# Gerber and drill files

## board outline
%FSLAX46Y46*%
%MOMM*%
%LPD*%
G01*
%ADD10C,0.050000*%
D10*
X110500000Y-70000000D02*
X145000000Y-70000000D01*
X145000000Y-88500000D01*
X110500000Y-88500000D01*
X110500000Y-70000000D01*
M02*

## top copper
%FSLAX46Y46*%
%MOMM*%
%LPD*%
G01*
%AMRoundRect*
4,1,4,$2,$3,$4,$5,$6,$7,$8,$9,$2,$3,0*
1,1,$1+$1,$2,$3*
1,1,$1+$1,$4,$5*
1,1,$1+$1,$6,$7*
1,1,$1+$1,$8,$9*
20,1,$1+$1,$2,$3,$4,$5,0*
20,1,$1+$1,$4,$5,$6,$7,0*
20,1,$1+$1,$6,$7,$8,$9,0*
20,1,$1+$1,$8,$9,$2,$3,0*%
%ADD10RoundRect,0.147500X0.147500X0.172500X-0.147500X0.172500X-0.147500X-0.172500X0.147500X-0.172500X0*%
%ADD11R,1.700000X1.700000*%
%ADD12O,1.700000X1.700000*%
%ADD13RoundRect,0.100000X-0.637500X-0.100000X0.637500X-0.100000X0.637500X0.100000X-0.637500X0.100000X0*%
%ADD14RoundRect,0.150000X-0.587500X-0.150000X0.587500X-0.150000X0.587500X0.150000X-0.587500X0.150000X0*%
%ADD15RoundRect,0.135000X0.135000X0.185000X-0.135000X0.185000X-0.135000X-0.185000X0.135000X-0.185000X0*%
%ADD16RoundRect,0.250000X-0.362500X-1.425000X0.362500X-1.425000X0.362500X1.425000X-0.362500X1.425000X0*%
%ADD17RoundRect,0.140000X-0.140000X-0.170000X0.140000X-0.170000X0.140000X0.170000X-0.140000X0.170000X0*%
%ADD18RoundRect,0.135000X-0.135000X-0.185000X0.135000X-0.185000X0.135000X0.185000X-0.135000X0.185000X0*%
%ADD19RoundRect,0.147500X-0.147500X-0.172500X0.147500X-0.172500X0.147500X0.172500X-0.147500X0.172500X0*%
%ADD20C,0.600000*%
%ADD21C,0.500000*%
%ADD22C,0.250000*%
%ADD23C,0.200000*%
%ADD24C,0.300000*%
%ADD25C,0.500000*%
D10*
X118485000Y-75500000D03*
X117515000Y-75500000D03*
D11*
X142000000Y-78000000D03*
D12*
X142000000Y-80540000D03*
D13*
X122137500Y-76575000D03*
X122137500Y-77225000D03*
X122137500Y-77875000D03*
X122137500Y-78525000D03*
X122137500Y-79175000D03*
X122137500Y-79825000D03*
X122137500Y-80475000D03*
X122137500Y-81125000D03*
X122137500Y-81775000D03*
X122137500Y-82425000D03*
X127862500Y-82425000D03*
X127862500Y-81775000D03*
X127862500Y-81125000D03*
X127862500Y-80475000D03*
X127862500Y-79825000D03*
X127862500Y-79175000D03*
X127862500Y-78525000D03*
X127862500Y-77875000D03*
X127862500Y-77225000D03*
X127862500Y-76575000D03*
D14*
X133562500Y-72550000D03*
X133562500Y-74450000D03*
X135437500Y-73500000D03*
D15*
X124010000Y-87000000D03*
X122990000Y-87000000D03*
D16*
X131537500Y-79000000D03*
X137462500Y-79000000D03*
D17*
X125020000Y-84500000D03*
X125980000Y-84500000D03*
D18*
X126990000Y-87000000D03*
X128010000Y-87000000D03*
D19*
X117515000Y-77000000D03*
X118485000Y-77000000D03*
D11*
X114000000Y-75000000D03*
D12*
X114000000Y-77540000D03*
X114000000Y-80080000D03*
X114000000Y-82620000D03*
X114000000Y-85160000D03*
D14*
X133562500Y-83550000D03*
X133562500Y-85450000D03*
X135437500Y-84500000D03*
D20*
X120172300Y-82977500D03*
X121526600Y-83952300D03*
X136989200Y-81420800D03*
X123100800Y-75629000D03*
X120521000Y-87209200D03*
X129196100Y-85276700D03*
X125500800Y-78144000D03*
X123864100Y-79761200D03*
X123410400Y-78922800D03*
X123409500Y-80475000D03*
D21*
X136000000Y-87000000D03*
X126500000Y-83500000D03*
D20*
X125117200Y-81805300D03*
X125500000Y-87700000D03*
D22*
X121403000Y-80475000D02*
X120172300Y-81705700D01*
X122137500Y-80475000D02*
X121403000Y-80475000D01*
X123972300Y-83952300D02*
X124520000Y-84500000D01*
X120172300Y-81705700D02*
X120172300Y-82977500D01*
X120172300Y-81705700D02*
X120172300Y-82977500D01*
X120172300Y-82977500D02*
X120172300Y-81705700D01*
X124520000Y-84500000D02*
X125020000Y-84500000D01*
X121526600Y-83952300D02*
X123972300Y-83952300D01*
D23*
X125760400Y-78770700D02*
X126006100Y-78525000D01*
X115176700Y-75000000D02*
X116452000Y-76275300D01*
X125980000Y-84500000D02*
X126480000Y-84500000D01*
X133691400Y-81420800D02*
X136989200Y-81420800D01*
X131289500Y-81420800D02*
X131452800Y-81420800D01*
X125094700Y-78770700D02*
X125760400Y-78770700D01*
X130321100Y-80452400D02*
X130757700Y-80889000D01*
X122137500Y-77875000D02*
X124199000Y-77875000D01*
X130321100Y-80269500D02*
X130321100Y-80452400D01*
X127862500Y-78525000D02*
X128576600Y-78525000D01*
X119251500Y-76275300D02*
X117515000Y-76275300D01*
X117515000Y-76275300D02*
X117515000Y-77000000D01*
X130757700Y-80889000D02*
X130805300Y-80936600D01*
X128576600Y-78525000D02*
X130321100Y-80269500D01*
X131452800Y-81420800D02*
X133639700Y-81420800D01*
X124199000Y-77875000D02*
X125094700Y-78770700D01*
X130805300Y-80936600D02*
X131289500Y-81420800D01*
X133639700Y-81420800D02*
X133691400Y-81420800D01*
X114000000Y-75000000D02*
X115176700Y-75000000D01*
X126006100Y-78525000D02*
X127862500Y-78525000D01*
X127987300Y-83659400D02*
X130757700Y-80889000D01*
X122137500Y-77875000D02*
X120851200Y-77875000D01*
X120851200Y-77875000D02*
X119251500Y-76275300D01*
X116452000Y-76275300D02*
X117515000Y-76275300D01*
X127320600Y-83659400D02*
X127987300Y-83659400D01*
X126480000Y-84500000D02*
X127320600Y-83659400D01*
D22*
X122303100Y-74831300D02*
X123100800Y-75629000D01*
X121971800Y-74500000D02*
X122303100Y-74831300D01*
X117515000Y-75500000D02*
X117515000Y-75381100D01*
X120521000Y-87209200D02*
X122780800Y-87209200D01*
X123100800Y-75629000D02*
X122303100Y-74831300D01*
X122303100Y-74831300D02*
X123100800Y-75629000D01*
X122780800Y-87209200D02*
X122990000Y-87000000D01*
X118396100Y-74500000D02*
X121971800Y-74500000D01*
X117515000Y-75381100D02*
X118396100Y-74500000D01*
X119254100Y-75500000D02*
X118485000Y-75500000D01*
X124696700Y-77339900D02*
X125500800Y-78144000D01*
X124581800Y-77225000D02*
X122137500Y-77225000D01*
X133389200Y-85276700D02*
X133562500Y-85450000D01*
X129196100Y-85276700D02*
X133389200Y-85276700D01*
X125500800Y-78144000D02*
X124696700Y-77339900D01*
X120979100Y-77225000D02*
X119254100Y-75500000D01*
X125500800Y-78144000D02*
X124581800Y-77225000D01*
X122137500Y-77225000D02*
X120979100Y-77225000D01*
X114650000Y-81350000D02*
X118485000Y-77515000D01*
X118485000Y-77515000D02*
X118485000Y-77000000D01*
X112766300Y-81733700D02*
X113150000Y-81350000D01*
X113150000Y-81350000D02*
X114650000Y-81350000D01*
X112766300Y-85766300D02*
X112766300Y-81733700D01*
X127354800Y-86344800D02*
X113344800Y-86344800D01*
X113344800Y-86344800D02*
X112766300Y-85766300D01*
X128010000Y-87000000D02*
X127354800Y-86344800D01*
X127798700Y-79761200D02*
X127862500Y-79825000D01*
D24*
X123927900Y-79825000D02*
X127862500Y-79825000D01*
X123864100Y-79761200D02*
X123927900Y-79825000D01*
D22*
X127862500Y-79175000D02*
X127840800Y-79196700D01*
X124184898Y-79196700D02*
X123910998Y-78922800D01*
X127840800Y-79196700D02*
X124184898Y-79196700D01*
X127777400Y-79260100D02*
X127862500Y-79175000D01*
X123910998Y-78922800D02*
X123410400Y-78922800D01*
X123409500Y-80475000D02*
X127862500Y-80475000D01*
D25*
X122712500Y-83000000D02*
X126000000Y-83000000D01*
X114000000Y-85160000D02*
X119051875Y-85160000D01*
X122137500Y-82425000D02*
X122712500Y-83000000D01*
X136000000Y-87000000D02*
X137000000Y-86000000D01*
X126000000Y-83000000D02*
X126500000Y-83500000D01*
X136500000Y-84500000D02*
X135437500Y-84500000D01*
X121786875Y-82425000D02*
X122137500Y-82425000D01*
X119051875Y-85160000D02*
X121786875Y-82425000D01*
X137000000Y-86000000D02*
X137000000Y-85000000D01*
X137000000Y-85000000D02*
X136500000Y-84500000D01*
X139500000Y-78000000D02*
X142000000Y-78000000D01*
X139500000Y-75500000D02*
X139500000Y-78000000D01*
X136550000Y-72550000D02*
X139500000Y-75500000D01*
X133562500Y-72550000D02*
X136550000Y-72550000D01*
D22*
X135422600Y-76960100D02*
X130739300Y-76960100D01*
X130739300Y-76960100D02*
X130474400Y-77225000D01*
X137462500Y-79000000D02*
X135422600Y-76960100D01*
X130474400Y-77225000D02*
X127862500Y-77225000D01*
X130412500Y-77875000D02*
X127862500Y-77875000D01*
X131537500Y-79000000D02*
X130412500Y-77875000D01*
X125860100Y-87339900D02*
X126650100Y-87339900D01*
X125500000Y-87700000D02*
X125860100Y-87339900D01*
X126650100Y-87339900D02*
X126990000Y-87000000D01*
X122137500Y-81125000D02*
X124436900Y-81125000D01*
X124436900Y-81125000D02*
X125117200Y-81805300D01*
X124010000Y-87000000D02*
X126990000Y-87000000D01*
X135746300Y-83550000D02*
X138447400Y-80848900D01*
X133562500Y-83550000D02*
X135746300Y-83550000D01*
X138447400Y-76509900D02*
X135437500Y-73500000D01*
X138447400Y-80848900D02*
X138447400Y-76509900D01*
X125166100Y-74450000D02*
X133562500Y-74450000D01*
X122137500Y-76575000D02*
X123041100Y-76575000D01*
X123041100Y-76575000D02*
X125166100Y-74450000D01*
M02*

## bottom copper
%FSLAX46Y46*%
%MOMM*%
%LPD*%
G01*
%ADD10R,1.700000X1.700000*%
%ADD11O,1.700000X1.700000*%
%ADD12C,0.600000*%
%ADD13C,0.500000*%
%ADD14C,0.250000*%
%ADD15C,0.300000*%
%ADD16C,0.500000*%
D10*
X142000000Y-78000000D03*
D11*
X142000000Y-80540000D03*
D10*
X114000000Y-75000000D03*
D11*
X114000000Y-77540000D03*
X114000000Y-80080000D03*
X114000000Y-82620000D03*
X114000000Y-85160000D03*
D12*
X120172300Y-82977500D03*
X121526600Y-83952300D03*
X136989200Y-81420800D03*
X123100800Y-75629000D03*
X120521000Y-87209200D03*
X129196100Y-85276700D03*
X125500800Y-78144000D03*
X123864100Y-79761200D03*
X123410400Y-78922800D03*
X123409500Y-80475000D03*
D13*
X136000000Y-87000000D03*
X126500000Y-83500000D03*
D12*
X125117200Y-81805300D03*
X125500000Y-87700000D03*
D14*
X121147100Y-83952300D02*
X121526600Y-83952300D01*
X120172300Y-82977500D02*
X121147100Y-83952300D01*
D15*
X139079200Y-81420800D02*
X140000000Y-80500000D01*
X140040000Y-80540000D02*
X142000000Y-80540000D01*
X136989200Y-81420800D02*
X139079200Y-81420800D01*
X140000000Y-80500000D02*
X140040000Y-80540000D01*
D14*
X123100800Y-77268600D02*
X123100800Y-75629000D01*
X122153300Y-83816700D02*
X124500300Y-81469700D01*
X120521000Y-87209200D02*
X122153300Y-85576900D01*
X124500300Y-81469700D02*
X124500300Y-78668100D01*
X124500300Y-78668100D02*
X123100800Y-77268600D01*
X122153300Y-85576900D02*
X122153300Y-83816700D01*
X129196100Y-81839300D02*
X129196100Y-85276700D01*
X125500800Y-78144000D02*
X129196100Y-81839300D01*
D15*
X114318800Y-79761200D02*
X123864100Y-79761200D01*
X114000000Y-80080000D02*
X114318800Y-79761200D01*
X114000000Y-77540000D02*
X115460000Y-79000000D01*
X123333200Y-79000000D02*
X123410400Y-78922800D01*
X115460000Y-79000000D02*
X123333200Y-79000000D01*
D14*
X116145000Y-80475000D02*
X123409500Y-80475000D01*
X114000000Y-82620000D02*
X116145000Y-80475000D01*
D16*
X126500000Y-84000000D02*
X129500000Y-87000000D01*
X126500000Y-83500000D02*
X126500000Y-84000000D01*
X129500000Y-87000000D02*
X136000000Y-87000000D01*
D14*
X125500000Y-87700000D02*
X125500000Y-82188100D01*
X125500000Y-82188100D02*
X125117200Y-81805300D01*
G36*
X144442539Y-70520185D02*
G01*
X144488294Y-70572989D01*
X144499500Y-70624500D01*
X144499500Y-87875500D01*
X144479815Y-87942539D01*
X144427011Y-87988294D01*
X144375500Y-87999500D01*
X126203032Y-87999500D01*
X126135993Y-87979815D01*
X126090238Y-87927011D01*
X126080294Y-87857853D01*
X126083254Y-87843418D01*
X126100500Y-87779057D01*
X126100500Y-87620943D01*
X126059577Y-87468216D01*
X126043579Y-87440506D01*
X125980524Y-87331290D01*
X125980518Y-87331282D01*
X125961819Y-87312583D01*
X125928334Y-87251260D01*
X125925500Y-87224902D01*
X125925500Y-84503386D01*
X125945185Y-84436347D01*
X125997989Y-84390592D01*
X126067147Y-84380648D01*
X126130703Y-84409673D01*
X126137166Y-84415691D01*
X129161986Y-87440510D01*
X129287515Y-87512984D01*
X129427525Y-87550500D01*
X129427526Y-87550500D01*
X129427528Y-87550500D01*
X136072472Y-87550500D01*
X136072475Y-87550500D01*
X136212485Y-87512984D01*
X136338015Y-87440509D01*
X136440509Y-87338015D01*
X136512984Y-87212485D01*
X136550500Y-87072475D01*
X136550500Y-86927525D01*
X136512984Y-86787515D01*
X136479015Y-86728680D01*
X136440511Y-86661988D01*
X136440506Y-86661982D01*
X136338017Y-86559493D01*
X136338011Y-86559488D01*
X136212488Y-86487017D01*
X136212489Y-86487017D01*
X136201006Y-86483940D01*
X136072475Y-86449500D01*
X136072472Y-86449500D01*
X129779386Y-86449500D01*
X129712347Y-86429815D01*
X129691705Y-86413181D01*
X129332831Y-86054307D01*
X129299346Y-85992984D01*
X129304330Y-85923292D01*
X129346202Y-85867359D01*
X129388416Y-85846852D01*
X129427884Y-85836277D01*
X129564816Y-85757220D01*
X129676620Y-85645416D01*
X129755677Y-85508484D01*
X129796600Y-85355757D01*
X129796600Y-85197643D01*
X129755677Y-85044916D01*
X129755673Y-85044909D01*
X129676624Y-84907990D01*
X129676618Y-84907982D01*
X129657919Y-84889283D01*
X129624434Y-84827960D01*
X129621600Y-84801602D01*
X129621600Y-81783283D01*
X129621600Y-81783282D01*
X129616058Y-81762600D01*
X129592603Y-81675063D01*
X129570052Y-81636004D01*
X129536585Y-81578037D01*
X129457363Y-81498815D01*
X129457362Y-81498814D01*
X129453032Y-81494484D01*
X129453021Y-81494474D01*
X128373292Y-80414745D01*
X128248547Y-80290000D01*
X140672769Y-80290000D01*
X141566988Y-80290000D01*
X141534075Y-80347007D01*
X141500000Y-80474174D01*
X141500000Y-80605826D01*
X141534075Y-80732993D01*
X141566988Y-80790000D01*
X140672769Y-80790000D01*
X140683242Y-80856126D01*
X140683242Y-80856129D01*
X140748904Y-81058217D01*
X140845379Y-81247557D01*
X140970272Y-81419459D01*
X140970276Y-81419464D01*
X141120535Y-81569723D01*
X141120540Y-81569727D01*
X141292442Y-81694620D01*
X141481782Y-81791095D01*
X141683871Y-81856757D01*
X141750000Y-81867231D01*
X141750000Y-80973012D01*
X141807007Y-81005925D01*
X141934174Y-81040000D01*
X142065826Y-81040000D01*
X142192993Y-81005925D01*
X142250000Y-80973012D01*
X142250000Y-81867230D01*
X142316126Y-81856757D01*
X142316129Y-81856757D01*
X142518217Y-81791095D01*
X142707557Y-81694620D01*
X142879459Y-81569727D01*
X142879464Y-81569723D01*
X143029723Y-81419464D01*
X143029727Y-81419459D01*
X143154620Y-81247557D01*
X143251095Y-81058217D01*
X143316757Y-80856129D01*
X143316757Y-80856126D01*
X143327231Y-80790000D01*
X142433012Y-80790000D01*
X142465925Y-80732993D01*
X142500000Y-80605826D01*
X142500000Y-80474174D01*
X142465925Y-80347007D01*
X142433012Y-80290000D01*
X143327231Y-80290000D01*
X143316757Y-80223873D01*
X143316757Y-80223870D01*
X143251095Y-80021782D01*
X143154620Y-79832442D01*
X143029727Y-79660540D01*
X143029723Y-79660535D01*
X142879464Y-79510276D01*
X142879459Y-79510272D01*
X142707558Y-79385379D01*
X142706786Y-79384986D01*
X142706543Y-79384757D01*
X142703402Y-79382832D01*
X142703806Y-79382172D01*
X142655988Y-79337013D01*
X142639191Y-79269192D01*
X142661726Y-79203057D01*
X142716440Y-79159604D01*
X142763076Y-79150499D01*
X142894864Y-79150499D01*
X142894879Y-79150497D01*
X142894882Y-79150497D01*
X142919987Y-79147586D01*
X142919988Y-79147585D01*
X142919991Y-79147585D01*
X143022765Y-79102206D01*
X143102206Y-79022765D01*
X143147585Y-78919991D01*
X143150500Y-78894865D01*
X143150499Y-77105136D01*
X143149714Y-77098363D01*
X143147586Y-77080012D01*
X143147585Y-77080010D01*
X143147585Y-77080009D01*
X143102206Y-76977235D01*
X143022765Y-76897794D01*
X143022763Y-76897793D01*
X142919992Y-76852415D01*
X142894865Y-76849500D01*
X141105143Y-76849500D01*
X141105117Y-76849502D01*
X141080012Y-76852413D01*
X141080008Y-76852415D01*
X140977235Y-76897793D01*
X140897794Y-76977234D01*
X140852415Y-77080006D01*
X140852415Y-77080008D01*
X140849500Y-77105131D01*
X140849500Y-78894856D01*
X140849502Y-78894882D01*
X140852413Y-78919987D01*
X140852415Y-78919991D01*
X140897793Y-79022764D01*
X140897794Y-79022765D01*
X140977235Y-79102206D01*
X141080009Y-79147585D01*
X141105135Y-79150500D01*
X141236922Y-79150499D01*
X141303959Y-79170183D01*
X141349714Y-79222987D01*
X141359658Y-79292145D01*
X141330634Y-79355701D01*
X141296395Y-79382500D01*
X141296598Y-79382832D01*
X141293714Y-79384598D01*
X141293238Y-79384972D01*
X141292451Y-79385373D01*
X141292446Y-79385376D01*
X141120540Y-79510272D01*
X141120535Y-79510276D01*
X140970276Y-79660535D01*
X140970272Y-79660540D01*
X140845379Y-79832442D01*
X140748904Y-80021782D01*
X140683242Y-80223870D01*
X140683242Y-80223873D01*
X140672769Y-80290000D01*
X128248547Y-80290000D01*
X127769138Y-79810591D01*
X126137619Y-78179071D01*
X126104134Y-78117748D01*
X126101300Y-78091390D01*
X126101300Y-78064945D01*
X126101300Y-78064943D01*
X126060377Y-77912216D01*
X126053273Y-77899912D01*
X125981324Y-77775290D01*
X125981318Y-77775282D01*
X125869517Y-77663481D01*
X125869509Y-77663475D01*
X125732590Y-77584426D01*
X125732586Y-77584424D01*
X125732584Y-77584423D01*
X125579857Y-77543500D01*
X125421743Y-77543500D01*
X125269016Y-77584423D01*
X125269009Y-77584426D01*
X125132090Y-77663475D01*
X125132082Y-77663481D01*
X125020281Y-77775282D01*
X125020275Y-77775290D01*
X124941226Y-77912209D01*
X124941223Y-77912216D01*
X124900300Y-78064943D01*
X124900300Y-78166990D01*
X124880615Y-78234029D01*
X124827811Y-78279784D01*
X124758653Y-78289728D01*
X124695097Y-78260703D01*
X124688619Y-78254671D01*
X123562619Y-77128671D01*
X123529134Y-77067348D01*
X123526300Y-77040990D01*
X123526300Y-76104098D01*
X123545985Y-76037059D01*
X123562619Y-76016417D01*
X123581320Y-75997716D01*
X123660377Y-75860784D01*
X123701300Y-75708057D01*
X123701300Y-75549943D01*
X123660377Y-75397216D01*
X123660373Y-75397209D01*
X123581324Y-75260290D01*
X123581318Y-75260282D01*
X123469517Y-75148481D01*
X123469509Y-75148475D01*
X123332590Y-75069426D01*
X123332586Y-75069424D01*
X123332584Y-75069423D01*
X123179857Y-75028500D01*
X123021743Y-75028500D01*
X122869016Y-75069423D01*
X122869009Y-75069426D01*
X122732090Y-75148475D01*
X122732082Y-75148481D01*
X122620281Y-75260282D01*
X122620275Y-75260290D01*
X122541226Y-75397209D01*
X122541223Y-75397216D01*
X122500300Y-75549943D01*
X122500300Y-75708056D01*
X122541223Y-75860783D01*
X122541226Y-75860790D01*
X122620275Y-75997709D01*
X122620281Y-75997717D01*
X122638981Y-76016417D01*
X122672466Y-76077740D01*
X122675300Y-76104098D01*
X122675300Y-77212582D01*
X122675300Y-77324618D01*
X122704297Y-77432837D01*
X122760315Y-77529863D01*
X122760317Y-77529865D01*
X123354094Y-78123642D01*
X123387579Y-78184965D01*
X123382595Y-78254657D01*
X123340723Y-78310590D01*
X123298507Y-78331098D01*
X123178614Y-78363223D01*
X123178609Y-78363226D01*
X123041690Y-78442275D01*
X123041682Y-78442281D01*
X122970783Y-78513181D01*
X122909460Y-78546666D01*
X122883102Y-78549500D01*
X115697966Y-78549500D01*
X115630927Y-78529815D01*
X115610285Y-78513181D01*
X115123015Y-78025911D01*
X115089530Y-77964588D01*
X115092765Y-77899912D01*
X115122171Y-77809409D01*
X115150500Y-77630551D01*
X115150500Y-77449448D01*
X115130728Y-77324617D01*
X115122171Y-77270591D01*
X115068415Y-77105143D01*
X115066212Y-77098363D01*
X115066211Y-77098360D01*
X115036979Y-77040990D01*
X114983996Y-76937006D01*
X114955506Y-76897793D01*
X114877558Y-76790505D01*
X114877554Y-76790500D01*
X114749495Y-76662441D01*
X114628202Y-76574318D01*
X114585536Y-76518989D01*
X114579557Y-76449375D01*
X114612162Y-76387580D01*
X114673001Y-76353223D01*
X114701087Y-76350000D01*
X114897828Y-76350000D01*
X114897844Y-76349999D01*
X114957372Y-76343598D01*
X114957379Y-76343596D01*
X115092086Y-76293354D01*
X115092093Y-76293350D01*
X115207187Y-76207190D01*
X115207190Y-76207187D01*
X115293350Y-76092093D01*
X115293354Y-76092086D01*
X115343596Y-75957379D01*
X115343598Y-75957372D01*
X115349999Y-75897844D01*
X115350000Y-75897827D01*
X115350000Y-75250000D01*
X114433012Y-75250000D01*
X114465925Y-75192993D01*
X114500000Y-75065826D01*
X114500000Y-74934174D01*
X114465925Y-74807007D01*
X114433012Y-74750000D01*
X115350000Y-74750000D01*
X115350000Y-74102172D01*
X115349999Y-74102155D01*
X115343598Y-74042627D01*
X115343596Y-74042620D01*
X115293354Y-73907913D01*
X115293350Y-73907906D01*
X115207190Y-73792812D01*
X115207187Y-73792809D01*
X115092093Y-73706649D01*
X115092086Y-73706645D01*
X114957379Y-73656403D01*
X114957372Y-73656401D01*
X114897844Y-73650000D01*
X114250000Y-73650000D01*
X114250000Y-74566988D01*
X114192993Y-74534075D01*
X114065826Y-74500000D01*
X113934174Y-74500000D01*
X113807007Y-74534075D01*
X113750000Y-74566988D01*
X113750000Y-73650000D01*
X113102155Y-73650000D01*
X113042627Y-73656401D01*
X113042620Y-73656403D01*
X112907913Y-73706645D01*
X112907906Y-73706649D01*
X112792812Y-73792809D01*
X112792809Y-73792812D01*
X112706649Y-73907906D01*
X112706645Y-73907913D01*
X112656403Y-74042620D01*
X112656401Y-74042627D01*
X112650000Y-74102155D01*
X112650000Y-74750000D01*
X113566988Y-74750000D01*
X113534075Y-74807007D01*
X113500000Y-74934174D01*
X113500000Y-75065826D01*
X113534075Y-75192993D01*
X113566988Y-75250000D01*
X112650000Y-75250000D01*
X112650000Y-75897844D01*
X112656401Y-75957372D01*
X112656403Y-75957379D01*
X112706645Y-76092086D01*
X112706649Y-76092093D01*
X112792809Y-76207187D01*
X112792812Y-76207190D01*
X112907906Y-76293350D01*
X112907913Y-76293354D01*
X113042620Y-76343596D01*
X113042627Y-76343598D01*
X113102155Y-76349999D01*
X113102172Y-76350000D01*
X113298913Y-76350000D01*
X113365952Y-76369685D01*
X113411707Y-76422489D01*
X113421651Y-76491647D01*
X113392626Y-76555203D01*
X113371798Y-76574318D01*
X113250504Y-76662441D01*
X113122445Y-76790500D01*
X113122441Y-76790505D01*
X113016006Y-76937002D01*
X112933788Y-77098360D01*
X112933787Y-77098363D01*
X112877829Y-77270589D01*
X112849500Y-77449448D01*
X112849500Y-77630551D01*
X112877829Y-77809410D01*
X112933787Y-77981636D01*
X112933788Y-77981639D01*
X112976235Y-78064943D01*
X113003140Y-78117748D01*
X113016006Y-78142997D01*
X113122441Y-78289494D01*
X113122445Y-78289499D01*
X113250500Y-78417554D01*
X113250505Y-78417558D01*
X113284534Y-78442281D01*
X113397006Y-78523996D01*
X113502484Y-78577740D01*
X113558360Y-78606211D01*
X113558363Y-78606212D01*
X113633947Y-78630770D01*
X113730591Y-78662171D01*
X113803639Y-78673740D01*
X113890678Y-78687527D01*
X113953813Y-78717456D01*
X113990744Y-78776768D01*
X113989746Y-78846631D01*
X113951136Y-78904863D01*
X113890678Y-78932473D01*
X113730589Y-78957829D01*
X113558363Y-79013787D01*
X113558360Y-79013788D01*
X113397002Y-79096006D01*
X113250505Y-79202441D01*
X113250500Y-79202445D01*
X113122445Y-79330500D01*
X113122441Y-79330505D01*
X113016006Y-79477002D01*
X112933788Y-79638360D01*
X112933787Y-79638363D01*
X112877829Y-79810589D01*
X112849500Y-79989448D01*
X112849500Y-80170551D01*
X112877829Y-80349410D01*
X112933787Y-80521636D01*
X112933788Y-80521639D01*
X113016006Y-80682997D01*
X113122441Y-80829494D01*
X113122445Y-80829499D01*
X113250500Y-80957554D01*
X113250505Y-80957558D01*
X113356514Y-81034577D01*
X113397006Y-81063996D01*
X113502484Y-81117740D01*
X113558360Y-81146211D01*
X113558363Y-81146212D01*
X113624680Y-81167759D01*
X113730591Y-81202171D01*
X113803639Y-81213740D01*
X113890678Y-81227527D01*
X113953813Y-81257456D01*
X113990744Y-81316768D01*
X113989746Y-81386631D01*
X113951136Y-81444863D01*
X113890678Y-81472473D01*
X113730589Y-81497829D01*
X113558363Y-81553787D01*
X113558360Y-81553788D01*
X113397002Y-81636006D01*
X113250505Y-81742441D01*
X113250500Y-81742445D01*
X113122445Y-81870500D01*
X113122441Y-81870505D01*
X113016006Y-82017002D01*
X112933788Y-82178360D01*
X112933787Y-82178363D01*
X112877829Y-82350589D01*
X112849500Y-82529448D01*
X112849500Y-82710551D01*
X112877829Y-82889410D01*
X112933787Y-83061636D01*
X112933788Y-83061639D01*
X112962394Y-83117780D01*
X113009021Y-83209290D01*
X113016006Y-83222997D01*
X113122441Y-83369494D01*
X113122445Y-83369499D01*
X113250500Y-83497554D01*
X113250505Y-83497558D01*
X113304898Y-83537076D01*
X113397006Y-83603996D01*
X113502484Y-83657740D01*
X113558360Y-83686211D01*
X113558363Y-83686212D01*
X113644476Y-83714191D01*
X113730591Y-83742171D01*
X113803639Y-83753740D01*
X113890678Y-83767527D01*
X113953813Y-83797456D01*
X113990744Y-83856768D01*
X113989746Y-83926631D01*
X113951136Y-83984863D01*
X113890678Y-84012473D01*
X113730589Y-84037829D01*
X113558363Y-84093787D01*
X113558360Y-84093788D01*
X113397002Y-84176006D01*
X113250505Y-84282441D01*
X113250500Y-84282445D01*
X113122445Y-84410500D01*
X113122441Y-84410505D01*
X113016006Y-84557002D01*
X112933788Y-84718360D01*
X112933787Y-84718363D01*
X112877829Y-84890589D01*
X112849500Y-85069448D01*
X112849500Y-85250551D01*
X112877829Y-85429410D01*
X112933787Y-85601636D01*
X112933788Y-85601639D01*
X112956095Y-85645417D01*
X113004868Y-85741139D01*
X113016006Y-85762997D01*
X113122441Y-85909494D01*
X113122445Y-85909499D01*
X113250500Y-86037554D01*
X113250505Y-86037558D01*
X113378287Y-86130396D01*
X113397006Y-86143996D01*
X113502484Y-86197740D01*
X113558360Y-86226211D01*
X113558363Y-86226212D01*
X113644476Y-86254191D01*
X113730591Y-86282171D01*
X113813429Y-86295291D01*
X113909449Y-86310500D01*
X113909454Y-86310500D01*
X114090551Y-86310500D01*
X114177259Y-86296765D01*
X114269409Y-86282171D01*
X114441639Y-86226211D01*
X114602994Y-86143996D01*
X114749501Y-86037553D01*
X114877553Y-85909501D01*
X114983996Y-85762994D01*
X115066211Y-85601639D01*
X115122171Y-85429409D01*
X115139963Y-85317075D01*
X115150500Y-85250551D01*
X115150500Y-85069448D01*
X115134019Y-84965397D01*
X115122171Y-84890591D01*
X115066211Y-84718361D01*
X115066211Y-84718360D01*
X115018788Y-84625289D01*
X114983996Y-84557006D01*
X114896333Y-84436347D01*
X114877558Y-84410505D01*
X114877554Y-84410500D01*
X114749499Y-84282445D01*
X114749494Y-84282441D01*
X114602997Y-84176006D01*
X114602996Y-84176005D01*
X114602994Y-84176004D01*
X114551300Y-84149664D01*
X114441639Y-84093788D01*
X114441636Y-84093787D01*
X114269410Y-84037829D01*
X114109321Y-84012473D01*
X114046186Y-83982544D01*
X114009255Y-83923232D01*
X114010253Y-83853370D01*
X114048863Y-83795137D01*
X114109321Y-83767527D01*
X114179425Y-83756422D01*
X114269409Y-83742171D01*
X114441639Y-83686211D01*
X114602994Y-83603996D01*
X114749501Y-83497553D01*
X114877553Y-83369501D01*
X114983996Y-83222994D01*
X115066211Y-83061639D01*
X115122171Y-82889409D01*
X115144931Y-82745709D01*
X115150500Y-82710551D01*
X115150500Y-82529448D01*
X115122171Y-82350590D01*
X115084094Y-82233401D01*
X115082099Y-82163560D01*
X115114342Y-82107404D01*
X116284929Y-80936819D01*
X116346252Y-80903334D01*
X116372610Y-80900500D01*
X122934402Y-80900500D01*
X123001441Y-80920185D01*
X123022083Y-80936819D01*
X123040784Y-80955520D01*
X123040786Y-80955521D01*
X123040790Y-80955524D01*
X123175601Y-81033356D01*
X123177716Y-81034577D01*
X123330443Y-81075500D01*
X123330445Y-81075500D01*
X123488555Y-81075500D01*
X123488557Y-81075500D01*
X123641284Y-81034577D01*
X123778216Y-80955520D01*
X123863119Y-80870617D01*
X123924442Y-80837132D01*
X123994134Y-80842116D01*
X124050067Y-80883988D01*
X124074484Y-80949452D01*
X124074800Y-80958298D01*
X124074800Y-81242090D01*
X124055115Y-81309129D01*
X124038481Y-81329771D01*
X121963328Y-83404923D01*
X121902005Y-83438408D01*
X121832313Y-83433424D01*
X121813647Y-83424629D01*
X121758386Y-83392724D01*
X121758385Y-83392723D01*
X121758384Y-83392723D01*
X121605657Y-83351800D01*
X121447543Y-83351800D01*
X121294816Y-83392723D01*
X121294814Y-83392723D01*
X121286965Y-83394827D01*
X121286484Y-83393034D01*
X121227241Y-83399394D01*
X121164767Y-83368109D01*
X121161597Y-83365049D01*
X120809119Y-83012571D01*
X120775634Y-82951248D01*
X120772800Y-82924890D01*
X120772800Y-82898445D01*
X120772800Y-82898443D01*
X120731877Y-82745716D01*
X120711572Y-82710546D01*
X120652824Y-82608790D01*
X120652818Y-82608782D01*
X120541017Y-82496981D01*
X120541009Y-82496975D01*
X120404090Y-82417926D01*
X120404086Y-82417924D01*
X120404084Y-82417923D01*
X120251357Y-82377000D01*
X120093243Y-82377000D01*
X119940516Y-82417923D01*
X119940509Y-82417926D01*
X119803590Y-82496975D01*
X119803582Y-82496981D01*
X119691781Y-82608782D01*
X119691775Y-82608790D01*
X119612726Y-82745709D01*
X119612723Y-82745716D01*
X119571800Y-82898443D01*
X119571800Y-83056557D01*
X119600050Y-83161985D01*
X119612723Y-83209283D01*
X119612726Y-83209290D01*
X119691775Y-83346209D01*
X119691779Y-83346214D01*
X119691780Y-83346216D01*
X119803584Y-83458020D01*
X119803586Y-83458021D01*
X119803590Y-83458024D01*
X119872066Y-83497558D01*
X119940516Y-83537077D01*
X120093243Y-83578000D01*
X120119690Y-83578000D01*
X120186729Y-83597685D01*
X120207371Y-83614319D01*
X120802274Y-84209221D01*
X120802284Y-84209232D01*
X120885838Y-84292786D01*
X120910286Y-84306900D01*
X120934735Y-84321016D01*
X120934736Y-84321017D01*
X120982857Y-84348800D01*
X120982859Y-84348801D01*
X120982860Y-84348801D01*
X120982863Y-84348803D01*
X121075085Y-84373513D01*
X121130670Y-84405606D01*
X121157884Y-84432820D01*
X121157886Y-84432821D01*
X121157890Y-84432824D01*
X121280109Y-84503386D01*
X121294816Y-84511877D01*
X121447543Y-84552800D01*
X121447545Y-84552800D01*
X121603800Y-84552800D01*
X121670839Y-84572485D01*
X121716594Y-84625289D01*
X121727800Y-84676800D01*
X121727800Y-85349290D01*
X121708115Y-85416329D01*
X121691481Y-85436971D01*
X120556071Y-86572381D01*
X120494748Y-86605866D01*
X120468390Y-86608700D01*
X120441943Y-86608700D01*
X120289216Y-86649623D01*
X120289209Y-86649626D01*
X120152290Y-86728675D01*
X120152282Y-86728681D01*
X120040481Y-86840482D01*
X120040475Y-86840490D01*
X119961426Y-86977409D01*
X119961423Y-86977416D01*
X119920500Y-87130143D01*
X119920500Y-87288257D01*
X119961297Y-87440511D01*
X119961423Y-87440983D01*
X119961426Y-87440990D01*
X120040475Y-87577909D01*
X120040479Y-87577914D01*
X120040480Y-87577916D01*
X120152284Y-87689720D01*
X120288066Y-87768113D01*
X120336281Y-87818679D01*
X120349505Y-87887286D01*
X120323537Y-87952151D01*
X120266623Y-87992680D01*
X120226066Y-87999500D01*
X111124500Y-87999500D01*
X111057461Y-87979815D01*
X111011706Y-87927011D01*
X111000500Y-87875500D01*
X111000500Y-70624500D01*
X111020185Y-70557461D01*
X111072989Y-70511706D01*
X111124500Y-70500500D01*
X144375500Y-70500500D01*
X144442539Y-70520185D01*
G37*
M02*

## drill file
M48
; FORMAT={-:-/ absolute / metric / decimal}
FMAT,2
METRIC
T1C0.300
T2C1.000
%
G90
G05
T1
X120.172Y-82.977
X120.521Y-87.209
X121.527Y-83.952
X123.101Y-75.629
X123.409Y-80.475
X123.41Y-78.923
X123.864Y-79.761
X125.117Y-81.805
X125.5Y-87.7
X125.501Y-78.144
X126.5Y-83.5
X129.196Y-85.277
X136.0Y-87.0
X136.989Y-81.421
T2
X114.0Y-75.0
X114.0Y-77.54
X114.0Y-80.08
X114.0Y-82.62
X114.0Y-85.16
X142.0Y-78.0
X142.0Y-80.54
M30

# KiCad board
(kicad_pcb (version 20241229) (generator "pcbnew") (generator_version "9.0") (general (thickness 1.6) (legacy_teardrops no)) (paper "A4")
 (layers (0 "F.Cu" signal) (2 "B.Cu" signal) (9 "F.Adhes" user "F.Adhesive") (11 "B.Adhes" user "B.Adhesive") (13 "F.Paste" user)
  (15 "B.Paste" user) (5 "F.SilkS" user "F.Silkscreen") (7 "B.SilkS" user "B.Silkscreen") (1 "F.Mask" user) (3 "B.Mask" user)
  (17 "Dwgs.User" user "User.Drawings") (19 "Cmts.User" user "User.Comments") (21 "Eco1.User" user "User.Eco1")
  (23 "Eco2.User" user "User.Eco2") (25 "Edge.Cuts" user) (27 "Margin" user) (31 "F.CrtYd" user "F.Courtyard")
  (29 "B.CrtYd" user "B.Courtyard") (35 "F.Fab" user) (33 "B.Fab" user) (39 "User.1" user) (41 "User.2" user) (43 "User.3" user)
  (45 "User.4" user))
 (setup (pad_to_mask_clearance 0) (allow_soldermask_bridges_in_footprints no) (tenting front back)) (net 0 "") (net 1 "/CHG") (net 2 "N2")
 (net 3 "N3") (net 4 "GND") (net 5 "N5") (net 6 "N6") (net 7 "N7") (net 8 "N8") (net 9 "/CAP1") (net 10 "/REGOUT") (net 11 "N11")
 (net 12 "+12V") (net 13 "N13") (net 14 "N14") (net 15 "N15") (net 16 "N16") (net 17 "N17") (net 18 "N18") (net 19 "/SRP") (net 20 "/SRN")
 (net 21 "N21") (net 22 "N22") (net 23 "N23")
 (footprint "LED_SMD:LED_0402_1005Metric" (layer "F.Cu") (at 118 75.5 180)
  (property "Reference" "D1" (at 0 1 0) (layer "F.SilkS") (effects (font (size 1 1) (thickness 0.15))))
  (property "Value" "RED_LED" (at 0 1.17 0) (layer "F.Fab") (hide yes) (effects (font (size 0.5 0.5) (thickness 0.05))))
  (pad "1" smd roundrect (at -0.485 0 180) (size 0.59 0.64) (layers "F.Cu" "F.Mask" "F.Paste") (roundrect_rratio 0.25) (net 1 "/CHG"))
  (pad "2" smd roundrect (at 0.485 0 180) (size 0.59 0.64) (layers "F.Cu" "F.Mask" "F.Paste") (roundrect_rratio 0.25) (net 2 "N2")))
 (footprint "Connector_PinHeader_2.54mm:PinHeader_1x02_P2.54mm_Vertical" (layer "F.Cu") (at 142 78)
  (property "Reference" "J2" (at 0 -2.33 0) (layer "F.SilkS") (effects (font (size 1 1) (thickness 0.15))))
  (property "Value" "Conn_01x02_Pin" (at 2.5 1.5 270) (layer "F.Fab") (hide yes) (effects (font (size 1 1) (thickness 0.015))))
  (pad "1" thru_hole rect (at 0 0) (size 1.7 1.7) (drill 1) (layers "*.Cu" "*.Mask") (remove_unused_layers no) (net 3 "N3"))
  (pad "2" thru_hole oval (at 0 2.54) (size 1.7 1.7) (drill 1) (layers "*.Cu" "*.Mask") (remove_unused_layers no) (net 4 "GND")))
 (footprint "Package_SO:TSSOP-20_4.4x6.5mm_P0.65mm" (layer "F.Cu") (at 125 79.5)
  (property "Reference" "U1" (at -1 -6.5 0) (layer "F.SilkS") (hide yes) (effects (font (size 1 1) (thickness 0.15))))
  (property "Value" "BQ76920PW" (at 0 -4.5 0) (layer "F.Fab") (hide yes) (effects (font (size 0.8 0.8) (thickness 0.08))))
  (pad "1" smd roundrect (at -2.8625 -2.925) (size 1.475 0.4) (layers "F.Cu" "F.Mask" "F.Paste") (roundrect_rratio 0.25) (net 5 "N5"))
  (pad "2" smd roundrect (at -2.8625 -2.275) (size 1.475 0.4) (layers "F.Cu" "F.Mask" "F.Paste") (roundrect_rratio 0.25) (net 1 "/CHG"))
  (pad "3" smd roundrect (at -2.8625 -1.625) (size 1.475 0.4) (layers "F.Cu" "F.Mask" "F.Paste") (roundrect_rratio 0.25) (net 4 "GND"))
  (pad "4" smd roundrect (at -2.8625 -0.975) (size 1.475 0.4) (layers "F.Cu" "F.Mask" "F.Paste") (roundrect_rratio 0.25) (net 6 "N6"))
  (pad "5" smd roundrect (at -2.8625 -0.325) (size 1.475 0.4) (layers "F.Cu" "F.Mask" "F.Paste") (roundrect_rratio 0.25) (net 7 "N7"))
  (pad "6" smd roundrect (at -2.8625 0.325) (size 1.475 0.4) (layers "F.Cu" "F.Mask" "F.Paste") (roundrect_rratio 0.25) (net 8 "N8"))
  (pad "7" smd roundrect (at -2.8625 0.975) (size 1.475 0.4) (layers "F.Cu" "F.Mask" "F.Paste") (roundrect_rratio 0.25) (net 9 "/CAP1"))
  (pad "8" smd roundrect (at -2.8625 1.625) (size 1.475 0.4) (layers "F.Cu" "F.Mask" "F.Paste") (roundrect_rratio 0.25) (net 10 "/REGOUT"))
  (pad "9" smd roundrect (at -2.8625 2.275) (size 1.475 0.4) (layers "F.Cu" "F.Mask" "F.Paste") (roundrect_rratio 0.25) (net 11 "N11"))
  (pad "10" smd roundrect (at -2.8625 2.925) (size 1.475 0.4) (layers "F.Cu" "F.Mask" "F.Paste") (roundrect_rratio 0.25) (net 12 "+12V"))
  (pad "11" smd roundrect (at 2.8625 2.925) (size 1.475 0.4) (layers "F.Cu" "F.Mask" "F.Paste") (roundrect_rratio 0.25) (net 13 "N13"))
  (pad "12" smd roundrect (at 2.8625 2.275) (size 1.475 0.4) (layers "F.Cu" "F.Mask" "F.Paste") (roundrect_rratio 0.25) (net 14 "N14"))
  (pad "13" smd roundrect (at 2.8625 1.625) (size 1.475 0.4) (layers "F.Cu" "F.Mask" "F.Paste") (roundrect_rratio 0.25) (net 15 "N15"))
  (pad "14" smd roundrect (at 2.8625 0.975) (size 1.475 0.4) (layers "F.Cu" "F.Mask" "F.Paste") (roundrect_rratio 0.25) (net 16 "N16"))
  (pad "15" smd roundrect (at 2.8625 0.325) (size 1.475 0.4) (layers "F.Cu" "F.Mask" "F.Paste") (roundrect_rratio 0.25) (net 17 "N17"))
  (pad "16" smd roundrect (at 2.8625 -0.325) (size 1.475 0.4) (layers "F.Cu" "F.Mask" "F.Paste") (roundrect_rratio 0.25) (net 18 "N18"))
  (pad "17" smd roundrect (at 2.8625 -0.975) (size 1.475 0.4) (layers "F.Cu" "F.Mask" "F.Paste") (roundrect_rratio 0.25) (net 4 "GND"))
  (pad "18" smd roundrect (at 2.8625 -1.625) (size 1.475 0.4) (layers "F.Cu" "F.Mask" "F.Paste") (roundrect_rratio 0.25) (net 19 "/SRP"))
  (pad "19" smd roundrect (at 2.8625 -2.275) (size 1.475 0.4) (layers "F.Cu" "F.Mask" "F.Paste") (roundrect_rratio 0.25) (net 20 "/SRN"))
  (pad "20" smd roundrect (at 2.8625 -2.925) (size 1.475 0.4) (layers "F.Cu" "F.Mask" "F.Paste") (roundrect_rratio 0.25) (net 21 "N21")))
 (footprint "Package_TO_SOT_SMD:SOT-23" (layer "F.Cu") (at 134.5 73.5)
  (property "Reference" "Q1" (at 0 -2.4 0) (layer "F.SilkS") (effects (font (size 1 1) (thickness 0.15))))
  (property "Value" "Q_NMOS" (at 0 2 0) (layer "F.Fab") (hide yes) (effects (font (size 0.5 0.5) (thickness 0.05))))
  (pad "1" smd roundrect (at -0.9375 -0.95) (size 1.475 0.6) (layers "F.Cu" "F.Mask" "F.Paste") (roundrect_rratio 0.25) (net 3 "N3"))
  (pad "2" smd roundrect (at -0.9375 0.95) (size 1.475 0.6) (layers "F.Cu" "F.Mask" "F.Paste") (roundrect_rratio 0.25) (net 5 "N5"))
  (pad "3" smd roundrect (at 0.9375 0) (size 1.475 0.6) (layers "F.Cu" "F.Mask" "F.Paste") (roundrect_rratio 0.25) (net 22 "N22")))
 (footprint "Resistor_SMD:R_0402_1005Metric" (layer "F.Cu") (at 123.5 87 180)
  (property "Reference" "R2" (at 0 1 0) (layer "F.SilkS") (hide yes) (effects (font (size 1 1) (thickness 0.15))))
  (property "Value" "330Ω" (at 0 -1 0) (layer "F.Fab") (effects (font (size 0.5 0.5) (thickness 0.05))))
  (pad "1" smd roundrect (at -0.51 0 180) (size 0.54 0.64) (layers "F.Cu" "F.Mask" "F.Paste") (roundrect_rratio 0.25) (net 10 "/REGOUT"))
  (pad "2" smd roundrect (at 0.51 0 180) (size 0.54 0.64) (layers "F.Cu" "F.Mask" "F.Paste") (roundrect_rratio 0.25) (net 2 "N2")))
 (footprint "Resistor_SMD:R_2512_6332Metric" (layer "F.Cu") (at 134.5 79)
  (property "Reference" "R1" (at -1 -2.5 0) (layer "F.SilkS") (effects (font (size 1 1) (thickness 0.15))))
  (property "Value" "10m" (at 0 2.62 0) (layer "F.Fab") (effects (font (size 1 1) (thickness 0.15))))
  (pad "1" smd roundrect (at -2.9625 0) (size 1.225 3.35) (layers "F.Cu" "F.Mask" "F.Paste") (roundrect_rratio 0.204082) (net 19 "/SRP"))
  (pad "2" smd roundrect (at 2.9625 0) (size 1.225 3.35) (layers "F.Cu" "F.Mask" "F.Paste") (roundrect_rratio 0.204082) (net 20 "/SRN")))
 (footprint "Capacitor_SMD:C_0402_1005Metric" (layer "F.Cu") (at 125.5 84.5)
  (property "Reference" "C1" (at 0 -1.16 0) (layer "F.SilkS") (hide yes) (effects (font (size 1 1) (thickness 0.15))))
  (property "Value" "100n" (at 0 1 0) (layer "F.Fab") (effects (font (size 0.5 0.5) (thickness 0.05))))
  (pad "1" smd roundrect (at -0.48 0) (size 0.56 0.62) (layers "F.Cu" "F.Mask" "F.Paste") (roundrect_rratio 0.25) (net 9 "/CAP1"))
  (pad "2" smd roundrect (at 0.48 0) (size 0.56 0.62) (layers "F.Cu" "F.Mask" "F.Paste") (roundrect_rratio 0.25) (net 4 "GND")))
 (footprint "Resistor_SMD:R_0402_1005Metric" (layer "F.Cu") (at 127.5 87)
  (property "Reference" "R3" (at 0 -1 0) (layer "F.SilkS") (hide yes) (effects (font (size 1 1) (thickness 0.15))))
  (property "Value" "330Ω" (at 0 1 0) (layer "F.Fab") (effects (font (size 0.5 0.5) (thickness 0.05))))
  (pad "1" smd roundrect (at -0.51 0) (size 0.54 0.64) (layers "F.Cu" "F.Mask" "F.Paste") (roundrect_rratio 0.25) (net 10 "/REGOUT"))
  (pad "2" smd roundrect (at 0.51 0) (size 0.54 0.64) (layers "F.Cu" "F.Mask" "F.Paste") (roundrect_rratio 0.25) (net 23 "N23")))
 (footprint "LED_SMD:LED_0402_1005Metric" (layer "F.Cu") (at 118 77)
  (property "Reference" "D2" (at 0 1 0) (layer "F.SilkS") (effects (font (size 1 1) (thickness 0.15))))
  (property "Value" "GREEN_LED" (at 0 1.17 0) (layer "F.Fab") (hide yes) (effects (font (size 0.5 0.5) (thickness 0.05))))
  (pad "1" smd roundrect (at -0.485 0) (size 0.59 0.64) (layers "F.Cu" "F.Mask" "F.Paste") (roundrect_rratio 0.25) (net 4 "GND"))
  (pad "2" smd roundrect (at 0.485 0) (size 0.59 0.64) (layers "F.Cu" "F.Mask" "F.Paste") (roundrect_rratio 0.25) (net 23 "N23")))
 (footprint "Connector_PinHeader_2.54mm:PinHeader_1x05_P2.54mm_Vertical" (layer "F.Cu") (at 114 75)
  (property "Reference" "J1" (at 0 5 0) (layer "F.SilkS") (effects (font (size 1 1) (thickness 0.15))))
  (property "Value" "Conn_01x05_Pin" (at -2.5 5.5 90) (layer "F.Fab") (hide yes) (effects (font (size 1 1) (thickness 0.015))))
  (pad "1" thru_hole rect (at 0 0) (size 1.7 1.7) (drill 1) (layers "*.Cu" "*.Mask") (remove_unused_layers no) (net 4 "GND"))
  (pad "2" thru_hole oval (at 0 2.54) (size 1.7 1.7) (drill 1) (layers "*.Cu" "*.Mask") (remove_unused_layers no) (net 18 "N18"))
  (pad "3" thru_hole oval (at 0 5.08) (size 1.7 1.7) (drill 1) (layers "*.Cu" "*.Mask") (remove_unused_layers no) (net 17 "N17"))
  (pad "4" thru_hole oval (at 0 7.62) (size 1.7 1.7) (drill 1) (layers "*.Cu" "*.Mask") (remove_unused_layers no) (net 16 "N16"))
  (pad "5" thru_hole oval (at 0 10.16) (size 1.7 1.7) (drill 1) (layers "*.Cu" "*.Mask") (remove_unused_layers no) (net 12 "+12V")))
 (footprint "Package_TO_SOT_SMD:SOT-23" (layer "F.Cu") (at 134.5 84.5)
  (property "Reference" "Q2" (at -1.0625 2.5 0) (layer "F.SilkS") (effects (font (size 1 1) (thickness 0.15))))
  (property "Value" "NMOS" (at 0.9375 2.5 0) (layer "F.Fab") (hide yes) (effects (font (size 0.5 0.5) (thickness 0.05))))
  (pad "1" smd roundrect (at -0.9375 -0.95) (size 1.475 0.6) (layers "F.Cu" "F.Mask" "F.Paste") (roundrect_rratio 0.25) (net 22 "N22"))
  (pad "2" smd roundrect (at -0.9375 0.95) (size 1.475 0.6) (layers "F.Cu" "F.Mask" "F.Paste") (roundrect_rratio 0.25) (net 1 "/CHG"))
  (pad "3" smd roundrect (at 0.9375 0) (size 1.475 0.6) (layers "F.Cu" "F.Mask" "F.Paste") (roundrect_rratio 0.25) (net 12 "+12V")))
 (gr_rect (start 110.5 70) (end 145 88.5) (stroke (width 0.05) (type solid)) (fill no) (layer "Edge.Cuts"))
 (segment (start 121.403 80.475) (end 120.1723 81.7057) (width 0.25) (layer "F.Cu") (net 9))
 (segment (start 122.1375 80.475) (end 121.403 80.475) (width 0.25) (layer "F.Cu") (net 9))
 (segment (start 123.9723 83.9523) (end 124.52 84.5) (width 0.25) (layer "F.Cu") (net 9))
 (segment (start 120.1723 81.7057) (end 120.1723 82.9775) (width 0.25) (layer "F.Cu") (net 9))
 (segment (start 120.1723 81.7057) (end 120.1723 82.9775) (width 0.25) (layer "F.Cu") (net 9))
 (segment (start 120.1723 82.9775) (end 120.1723 81.7057) (width 0.25) (layer "F.Cu") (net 9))
 (segment (start 124.52 84.5) (end 125.02 84.5) (width 0.25) (layer "F.Cu") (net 9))
 (segment (start 121.5266 83.9523) (end 123.9723 83.9523) (width 0.25) (layer "F.Cu") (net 9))
 (via (at 120.1723 82.9775) (size 0.6) (drill 0.3) (layers "F.Cu" "B.Cu") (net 9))
 (via (at 121.5266 83.9523) (size 0.6) (drill 0.3) (layers "F.Cu" "B.Cu") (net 9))
 (segment (start 121.1471 83.9523) (end 121.5266 83.9523) (width 0.25) (layer "B.Cu") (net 9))
 (segment (start 120.1723 82.9775) (end 121.1471 83.9523) (width 0.25) (layer "B.Cu") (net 9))
 (segment (start 125.7604 78.7707) (end 126.0061 78.525) (width 0.2) (layer "F.Cu") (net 4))
 (segment (start 115.1767 75) (end 116.452 76.2753) (width 0.2) (layer "F.Cu") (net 4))
 (segment (start 125.98 84.5) (end 126.48 84.5) (width 0.2) (layer "F.Cu") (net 4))
 (segment (start 133.6914 81.4208) (end 136.9892 81.4208) (width 0.2) (layer "F.Cu") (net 4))
 (segment (start 131.2895 81.4208) (end 131.4528 81.4208) (width 0.2) (layer "F.Cu") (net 4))
 (segment (start 125.0947 78.7707) (end 125.7604 78.7707) (width 0.2) (layer "F.Cu") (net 4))
 (segment (start 130.3211 80.4524) (end 130.7577 80.889) (width 0.2) (layer "F.Cu") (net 4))
 (segment (start 122.1375 77.875) (end 124.199 77.875) (width 0.2) (layer "F.Cu") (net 4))
 (segment (start 130.3211 80.2695) (end 130.3211 80.4524) (width 0.2) (layer "F.Cu") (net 4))
 (segment (start 127.8625 78.525) (end 128.5766 78.525) (width 0.2) (layer "F.Cu") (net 4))
 (segment (start 119.2515 76.2753) (end 117.515 76.2753) (width 0.2) (layer "F.Cu") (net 4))
 (segment (start 117.515 76.2753) (end 117.515 77) (width 0.2) (layer "F.Cu") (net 4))
 (segment (start 130.7577 80.889) (end 130.8053 80.9366) (width 0.2) (layer "F.Cu") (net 4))
 (segment (start 128.5766 78.525) (end 130.3211 80.2695) (width 0.2) (layer "F.Cu") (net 4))
 (segment (start 131.4528 81.4208) (end 133.6397 81.4208) (width 0.2) (layer "F.Cu") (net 4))
 (segment (start 124.199 77.875) (end 125.0947 78.7707) (width 0.2) (layer "F.Cu") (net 4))
 (segment (start 130.8053 80.9366) (end 131.2895 81.4208) (width 0.2) (layer "F.Cu") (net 4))
 (segment (start 133.6397 81.4208) (end 133.6914 81.4208) (width 0.2) (layer "F.Cu") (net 4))
 (segment (start 114 75) (end 115.1767 75) (width 0.2) (layer "F.Cu") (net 4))
 (segment (start 126.0061 78.525) (end 127.8625 78.525) (width 0.2) (layer "F.Cu") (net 4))
 (segment (start 127.9873 83.6594) (end 130.7577 80.889) (width 0.2) (layer "F.Cu") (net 4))
 (segment (start 122.1375 77.875) (end 120.8512 77.875) (width 0.2) (layer "F.Cu") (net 4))
 (segment (start 120.8512 77.875) (end 119.2515 76.2753) (width 0.2) (layer "F.Cu") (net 4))
 (segment (start 116.452 76.2753) (end 117.515 76.2753) (width 0.2) (layer "F.Cu") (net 4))
 (segment (start 127.3206 83.6594) (end 127.9873 83.6594) (width 0.2) (layer "F.Cu") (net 4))
 (segment (start 126.48 84.5) (end 127.3206 83.6594) (width 0.2) (layer "F.Cu") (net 4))
 (via (at 136.9892 81.4208) (size 0.6) (drill 0.3) (layers "F.Cu" "B.Cu") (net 4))
 (segment (start 139.0792 81.4208) (end 140 80.5) (width 0.3) (layer "B.Cu") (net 4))
 (segment (start 140.04 80.54) (end 142 80.54) (width 0.3) (layer "B.Cu") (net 4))
 (segment (start 136.9892 81.4208) (end 139.0792 81.4208) (width 0.3) (layer "B.Cu") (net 4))
 (segment (start 140 80.5) (end 140.04 80.54) (width 0.3) (layer "B.Cu") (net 4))
 (segment (start 122.3031 74.8313) (end 123.1008 75.629) (width 0.25) (layer "F.Cu") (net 2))
 (segment (start 121.9718 74.5) (end 122.3031 74.8313) (width 0.25) (layer "F.Cu") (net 2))
 (segment (start 117.515 75.5) (end 117.515 75.3811) (width 0.25) (layer "F.Cu") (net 2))
 (segment (start 120.521 87.2092) (end 122.7808 87.2092) (width 0.25) (layer "F.Cu") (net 2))
 (segment (start 123.1008 75.629) (end 122.3031 74.8313) (width 0.25) (layer "F.Cu") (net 2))
 (segment (start 122.3031 74.8313) (end 123.1008 75.629) (width 0.25) (layer "F.Cu") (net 2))
 (segment (start 122.7808 87.2092) (end 122.99 87) (width 0.25) (layer "F.Cu") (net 2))
 (segment (start 118.3961 74.5) (end 121.9718 74.5) (width 0.25) (layer "F.Cu") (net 2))
 (segment (start 117.515 75.3811) (end 118.3961 74.5) (width 0.25) (layer "F.Cu") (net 2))
 (via (at 123.1008 75.629) (size 0.6) (drill 0.3) (layers "F.Cu" "B.Cu") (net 2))
 (via (at 120.521 87.2092) (size 0.6) (drill 0.3) (layers "F.Cu" "B.Cu") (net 2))
 (segment (start 123.1008 77.2686) (end 123.1008 75.629) (width 0.25) (layer "B.Cu") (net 2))
 (segment (start 122.1533 83.8167) (end 124.5003 81.4697) (width 0.25) (layer "B.Cu") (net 2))
 (segment (start 120.521 87.2092) (end 122.1533 85.5769) (width 0.25) (layer "B.Cu") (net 2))
 (segment (start 124.5003 81.4697) (end 124.5003 78.6681) (width 0.25) (layer "B.Cu") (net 2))
 (segment (start 124.5003 78.6681) (end 123.1008 77.2686) (width 0.25) (layer "B.Cu") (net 2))
 (segment (start 122.1533 85.5769) (end 122.1533 83.8167) (width 0.25) (layer "B.Cu") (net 2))
 (segment (start 119.2541 75.5) (end 118.485 75.5) (width 0.25) (layer "F.Cu") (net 1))
 (segment (start 124.6967 77.3399) (end 125.5008 78.144) (width 0.25) (layer "F.Cu") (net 1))
 (segment (start 124.5818 77.225) (end 122.1375 77.225) (width 0.25) (layer "F.Cu") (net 1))
 (segment (start 133.3892 85.2767) (end 133.5625 85.45) (width 0.25) (layer "F.Cu") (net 1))
 (segment (start 129.1961 85.2767) (end 133.3892 85.2767) (width 0.25) (layer "F.Cu") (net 1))
 (segment (start 125.5008 78.144) (end 124.6967 77.3399) (width 0.25) (layer "F.Cu") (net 1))
 (segment (start 120.9791 77.225) (end 119.2541 75.5) (width 0.25) (layer "F.Cu") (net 1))
 (segment (start 125.5008 78.144) (end 124.5818 77.225) (width 0.25) (layer "F.Cu") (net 1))
 (segment (start 122.1375 77.225) (end 120.9791 77.225) (width 0.25) (layer "F.Cu") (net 1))
 (via (at 129.1961 85.2767) (size 0.6) (drill 0.3) (layers "F.Cu" "B.Cu") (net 1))
 (via (at 125.5008 78.144) (size 0.6) (drill 0.3) (layers "F.Cu" "B.Cu") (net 1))
 (segment (start 129.1961 81.8393) (end 129.1961 85.2767) (width 0.25) (layer "B.Cu") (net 1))
 (segment (start 125.5008 78.144) (end 129.1961 81.8393) (width 0.25) (layer "B.Cu") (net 1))
 (segment (start 114.65 81.35) (end 118.485 77.515) (width 0.25) (layer "F.Cu") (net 23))
 (segment (start 118.485 77.515) (end 118.485 77) (width 0.25) (layer "F.Cu") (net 23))
 (segment (start 112.7663 81.7337) (end 113.15 81.35) (width 0.25) (layer "F.Cu") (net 23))
 (segment (start 113.15 81.35) (end 114.65 81.35) (width 0.25) (layer "F.Cu") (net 23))
 (segment (start 112.7663 85.7663) (end 112.7663 81.7337) (width 0.25) (layer "F.Cu") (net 23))
 (segment (start 127.3548 86.3448) (end 113.3448 86.3448) (width 0.25) (layer "F.Cu") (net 23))
 (segment (start 113.3448 86.3448) (end 112.7663 85.7663) (width 0.25) (layer "F.Cu") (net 23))
 (segment (start 128.01 87) (end 127.3548 86.3448) (width 0.25) (layer "F.Cu") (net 23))
 (segment (start 127.7987 79.7612) (end 127.8625 79.825) (width 0.25) (layer "F.Cu") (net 17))
 (segment (start 123.9279 79.825) (end 127.8625 79.825) (width 0.3) (layer "F.Cu") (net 17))
 (segment (start 123.8641 79.7612) (end 123.9279 79.825) (width 0.3) (layer "F.Cu") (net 17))
 (via (at 123.8641 79.7612) (size 0.6) (drill 0.3) (layers "F.Cu" "B.Cu") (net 17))
 (segment (start 114.3188 79.7612) (end 123.8641 79.7612) (width 0.3) (layer "B.Cu") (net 17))
 (segment (start 114 80.08) (end 114.3188 79.7612) (width 0.3) (layer "B.Cu") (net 17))
 (segment (start 127.8625 79.175) (end 127.8408 79.1967) (width 0.25) (layer "F.Cu") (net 18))
 (segment (start 124.184898 79.1967) (end 123.910998 78.9228) (width 0.25) (layer "F.Cu") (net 18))
 (segment (start 127.8408 79.1967) (end 124.184898 79.1967) (width 0.25) (layer "F.Cu") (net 18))
 (segment (start 127.7774 79.2601) (end 127.8625 79.175) (width 0.25) (layer "F.Cu") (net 18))
 (segment (start 123.910998 78.9228) (end 123.4104 78.9228) (width 0.25) (layer "F.Cu") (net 18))
 (via (at 123.4104 78.9228) (size 0.6) (drill 0.3) (layers "F.Cu" "B.Cu") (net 18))
 (segment (start 114 77.54) (end 115.46 79) (width 0.3) (layer "B.Cu") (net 18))
 (segment (start 123.3332 79) (end 123.4104 78.9228) (width 0.3) (layer "B.Cu") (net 18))
 (segment (start 115.46 79) (end 123.3332 79) (width 0.3) (layer "B.Cu") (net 18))
 (segment (start 123.4095 80.475) (end 127.8625 80.475) (width 0.25) (layer "F.Cu") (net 16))
 (via (at 123.4095 80.475) (size 0.6) (drill 0.3) (layers "F.Cu" "B.Cu") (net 16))
 (segment (start 116.145 80.475) (end 123.4095 80.475) (width 0.25) (layer "B.Cu") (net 16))
 (segment (start 114 82.62) (end 116.145 80.475) (width 0.25) (layer "B.Cu") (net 16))
 (segment (start 122.7125 83) (end 126 83) (width 0.5) (layer "F.Cu") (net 12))
 (segment (start 114 85.16) (end 119.051875 85.16) (width 0.5) (layer "F.Cu") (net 12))
 (segment (start 122.1375 82.425) (end 122.7125 83) (width 0.5) (layer "F.Cu") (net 12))
 (segment (start 136 87) (end 137 86) (width 0.5) (layer "F.Cu") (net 12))
 (segment (start 126 83) (end 126.5 83.5) (width 0.5) (layer "F.Cu") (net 12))
 (segment (start 136.5 84.5) (end 135.4375 84.5) (width 0.5) (layer "F.Cu") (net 12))
 (segment (start 121.786875 82.425) (end 122.1375 82.425) (width 0.5) (layer "F.Cu") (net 12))
 (segment (start 119.051875 85.16) (end 121.786875 82.425) (width 0.5) (layer "F.Cu") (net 12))
 (segment (start 137 86) (end 137 85) (width 0.5) (layer "F.Cu") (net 12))
 (segment (start 137 85) (end 136.5 84.5) (width 0.5) (layer "F.Cu") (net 12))
 (via (at 136 87) (size 0.5) (drill 0.3) (layers "F.Cu" "B.Cu") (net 12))
 (via (at 126.5 83.5) (size 0.5) (drill 0.3) (layers "F.Cu" "B.Cu") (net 12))
 (segment (start 126.5 84) (end 129.5 87) (width 0.5) (layer "B.Cu") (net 12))
 (segment (start 126.5 83.5) (end 126.5 84) (width 0.5) (layer "B.Cu") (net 12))
 (segment (start 129.5 87) (end 136 87) (width 0.5) (layer "B.Cu") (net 12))
 (segment (start 139.5 78) (end 142 78) (width 0.5) (layer "F.Cu") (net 3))
 (segment (start 139.5 75.5) (end 139.5 78) (width 0.5) (layer "F.Cu") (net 3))
 (segment (start 136.55 72.55) (end 139.5 75.5) (width 0.5) (layer "F.Cu") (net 3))
 (segment (start 133.5625 72.55) (end 136.55 72.55) (width 0.5) (layer "F.Cu") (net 3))
 (segment (start 135.4226 76.9601) (end 130.7393 76.9601) (width 0.25) (layer "F.Cu") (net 20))
 (segment (start 130.7393 76.9601) (end 130.4744 77.225) (width 0.25) (layer "F.Cu") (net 20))
 (segment (start 137.4625 79) (end 135.4226 76.9601) (width 0.25) (layer "F.Cu") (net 20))
 (segment (start 130.4744 77.225) (end 127.8625 77.225) (width 0.25) (layer "F.Cu") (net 20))
 (segment (start 130.4125 77.875) (end 127.8625 77.875) (width 0.25) (layer "F.Cu") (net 19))
 (segment (start 131.5375 79) (end 130.4125 77.875) (width 0.25) (layer "F.Cu") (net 19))
 (segment (start 125.8601 87.3399) (end 126.6501 87.3399) (width 0.25) (layer "F.Cu") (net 10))
 (segment (start 125.5 87.7) (end 125.8601 87.3399) (width 0.25) (layer "F.Cu") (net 10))
 (segment (start 126.6501 87.3399) (end 126.99 87) (width 0.25) (layer "F.Cu") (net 10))
 (segment (start 122.1375 81.125) (end 124.4369 81.125) (width 0.25) (layer "F.Cu") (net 10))
 (segment (start 124.4369 81.125) (end 125.1172 81.8053) (width 0.25) (layer "F.Cu") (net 10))
 (segment (start 124.01 87) (end 126.99 87) (width 0.25) (layer "F.Cu") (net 10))
 (via (at 125.1172 81.8053) (size 0.6) (drill 0.3) (layers "F.Cu" "B.Cu") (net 10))
 (via (at 125.5 87.7) (size 0.6) (drill 0.3) (layers "F.Cu" "B.Cu") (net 10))
 (segment (start 125.5 87.7) (end 125.5 82.1881) (width 0.25) (layer "B.Cu") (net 10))
 (segment (start 125.5 82.1881) (end 125.1172 81.8053) (width 0.25) (layer "B.Cu") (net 10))
 (segment (start 135.7463 83.55) (end 138.4474 80.8489) (width 0.25) (layer "F.Cu") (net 22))
 (segment (start 133.5625 83.55) (end 135.7463 83.55) (width 0.25) (layer "F.Cu") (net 22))
 (segment (start 138.4474 76.5099) (end 135.4375 73.5) (width 0.25) (layer "F.Cu") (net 22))
 (segment (start 138.4474 80.8489) (end 138.4474 76.5099) (width 0.25) (layer "F.Cu") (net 22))
 (segment (start 125.1661 74.45) (end 133.5625 74.45) (width 0.25) (layer "F.Cu") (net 5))
 (segment (start 122.1375 76.575) (end 123.0411 76.575) (width 0.25) (layer "F.Cu") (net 5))
 (segment (start 123.0411 76.575) (end 125.1661 74.45) (width 0.25) (layer "F.Cu") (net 5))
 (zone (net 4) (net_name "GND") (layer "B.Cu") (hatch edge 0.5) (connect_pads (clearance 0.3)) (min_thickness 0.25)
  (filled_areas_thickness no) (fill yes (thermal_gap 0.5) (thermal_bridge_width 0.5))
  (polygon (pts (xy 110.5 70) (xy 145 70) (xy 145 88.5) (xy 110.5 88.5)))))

